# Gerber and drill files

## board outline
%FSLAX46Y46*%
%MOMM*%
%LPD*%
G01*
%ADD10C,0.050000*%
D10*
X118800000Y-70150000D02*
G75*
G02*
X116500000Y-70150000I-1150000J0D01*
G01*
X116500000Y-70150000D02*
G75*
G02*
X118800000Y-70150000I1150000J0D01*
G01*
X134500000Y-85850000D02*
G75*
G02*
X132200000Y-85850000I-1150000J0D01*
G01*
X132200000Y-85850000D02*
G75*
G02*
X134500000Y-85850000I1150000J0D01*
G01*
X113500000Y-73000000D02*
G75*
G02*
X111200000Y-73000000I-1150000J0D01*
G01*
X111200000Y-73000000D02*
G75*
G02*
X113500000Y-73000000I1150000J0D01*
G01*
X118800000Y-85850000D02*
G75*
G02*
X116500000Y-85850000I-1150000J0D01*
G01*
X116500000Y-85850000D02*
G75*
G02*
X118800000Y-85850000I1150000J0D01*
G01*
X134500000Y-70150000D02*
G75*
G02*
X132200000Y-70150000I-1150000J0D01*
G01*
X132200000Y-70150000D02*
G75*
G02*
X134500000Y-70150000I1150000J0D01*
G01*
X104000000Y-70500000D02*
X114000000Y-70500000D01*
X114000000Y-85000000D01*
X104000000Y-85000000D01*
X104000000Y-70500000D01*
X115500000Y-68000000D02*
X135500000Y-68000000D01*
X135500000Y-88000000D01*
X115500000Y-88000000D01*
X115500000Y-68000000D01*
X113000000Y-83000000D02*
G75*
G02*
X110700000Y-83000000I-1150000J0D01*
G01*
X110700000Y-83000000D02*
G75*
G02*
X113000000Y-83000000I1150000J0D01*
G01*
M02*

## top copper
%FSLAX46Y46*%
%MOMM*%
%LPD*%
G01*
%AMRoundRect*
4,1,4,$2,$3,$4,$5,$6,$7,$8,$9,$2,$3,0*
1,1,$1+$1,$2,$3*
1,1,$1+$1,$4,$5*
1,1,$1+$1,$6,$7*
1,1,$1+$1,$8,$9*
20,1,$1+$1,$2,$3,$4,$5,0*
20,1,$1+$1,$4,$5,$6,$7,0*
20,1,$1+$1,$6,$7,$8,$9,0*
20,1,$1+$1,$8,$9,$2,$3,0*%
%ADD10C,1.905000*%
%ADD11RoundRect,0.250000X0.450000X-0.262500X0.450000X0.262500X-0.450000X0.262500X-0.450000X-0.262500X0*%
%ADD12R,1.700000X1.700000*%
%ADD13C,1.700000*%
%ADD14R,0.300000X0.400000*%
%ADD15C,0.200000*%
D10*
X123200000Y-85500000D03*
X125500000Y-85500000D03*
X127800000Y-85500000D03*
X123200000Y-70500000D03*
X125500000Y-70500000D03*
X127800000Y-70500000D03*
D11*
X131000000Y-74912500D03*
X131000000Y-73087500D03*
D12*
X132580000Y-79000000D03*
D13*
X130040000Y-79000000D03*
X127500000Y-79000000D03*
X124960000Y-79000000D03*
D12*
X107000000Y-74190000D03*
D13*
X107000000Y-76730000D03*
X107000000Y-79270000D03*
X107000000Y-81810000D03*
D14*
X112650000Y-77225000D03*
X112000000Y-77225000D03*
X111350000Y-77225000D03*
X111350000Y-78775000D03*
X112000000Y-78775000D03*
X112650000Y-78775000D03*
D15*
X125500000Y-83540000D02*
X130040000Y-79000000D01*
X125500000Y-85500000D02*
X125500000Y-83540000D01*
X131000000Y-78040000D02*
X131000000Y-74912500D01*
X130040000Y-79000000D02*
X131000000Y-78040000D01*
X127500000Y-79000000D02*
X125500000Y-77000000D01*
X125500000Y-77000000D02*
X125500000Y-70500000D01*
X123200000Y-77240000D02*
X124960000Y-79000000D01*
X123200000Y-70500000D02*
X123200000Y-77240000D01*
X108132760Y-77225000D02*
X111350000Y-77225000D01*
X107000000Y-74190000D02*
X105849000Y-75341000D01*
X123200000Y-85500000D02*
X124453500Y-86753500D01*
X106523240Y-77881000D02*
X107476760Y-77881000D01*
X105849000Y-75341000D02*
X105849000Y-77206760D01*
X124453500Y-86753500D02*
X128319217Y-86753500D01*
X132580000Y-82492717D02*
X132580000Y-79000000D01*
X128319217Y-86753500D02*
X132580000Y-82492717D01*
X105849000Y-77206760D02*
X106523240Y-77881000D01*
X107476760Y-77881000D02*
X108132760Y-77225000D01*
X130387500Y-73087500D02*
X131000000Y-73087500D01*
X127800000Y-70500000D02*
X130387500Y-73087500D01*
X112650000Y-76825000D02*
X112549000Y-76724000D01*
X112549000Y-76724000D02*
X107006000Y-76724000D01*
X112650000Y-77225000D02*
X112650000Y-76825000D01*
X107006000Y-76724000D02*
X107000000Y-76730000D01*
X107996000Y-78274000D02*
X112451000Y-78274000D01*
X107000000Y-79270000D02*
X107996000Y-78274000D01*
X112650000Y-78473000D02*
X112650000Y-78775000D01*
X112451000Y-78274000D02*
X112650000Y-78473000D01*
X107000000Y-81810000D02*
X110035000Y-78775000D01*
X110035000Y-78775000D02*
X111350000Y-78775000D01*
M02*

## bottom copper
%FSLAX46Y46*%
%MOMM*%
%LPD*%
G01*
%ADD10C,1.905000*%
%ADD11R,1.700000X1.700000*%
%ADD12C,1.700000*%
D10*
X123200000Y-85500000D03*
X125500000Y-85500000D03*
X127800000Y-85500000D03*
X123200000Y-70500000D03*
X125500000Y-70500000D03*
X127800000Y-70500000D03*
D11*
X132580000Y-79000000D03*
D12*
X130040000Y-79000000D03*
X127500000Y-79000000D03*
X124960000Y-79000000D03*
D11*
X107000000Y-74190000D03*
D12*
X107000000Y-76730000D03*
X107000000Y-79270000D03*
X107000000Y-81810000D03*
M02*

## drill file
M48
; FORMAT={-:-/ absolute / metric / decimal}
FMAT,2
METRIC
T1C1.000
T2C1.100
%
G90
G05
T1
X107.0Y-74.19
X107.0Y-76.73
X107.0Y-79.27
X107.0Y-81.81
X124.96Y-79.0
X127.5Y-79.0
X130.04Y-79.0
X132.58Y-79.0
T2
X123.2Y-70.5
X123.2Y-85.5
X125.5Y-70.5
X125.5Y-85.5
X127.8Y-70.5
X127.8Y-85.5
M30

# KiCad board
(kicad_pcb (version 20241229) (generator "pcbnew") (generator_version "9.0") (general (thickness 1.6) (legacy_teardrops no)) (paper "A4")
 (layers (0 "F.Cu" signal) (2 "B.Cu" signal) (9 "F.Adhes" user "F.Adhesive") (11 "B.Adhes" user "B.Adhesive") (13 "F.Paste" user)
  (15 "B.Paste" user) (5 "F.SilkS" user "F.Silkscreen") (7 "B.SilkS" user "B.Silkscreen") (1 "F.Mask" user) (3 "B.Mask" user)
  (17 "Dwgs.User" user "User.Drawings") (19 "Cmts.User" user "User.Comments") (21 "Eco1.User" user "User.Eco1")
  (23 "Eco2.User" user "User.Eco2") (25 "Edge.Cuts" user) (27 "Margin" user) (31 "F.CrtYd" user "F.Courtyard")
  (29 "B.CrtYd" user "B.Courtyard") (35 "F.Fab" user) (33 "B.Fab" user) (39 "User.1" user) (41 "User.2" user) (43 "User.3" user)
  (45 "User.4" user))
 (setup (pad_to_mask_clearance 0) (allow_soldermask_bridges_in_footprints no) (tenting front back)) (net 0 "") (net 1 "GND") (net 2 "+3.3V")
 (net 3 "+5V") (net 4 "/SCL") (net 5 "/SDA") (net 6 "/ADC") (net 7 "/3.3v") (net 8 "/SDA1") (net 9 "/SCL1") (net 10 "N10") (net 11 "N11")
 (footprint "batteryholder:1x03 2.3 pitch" (layer "F.Cu") (at 123.4 85.5)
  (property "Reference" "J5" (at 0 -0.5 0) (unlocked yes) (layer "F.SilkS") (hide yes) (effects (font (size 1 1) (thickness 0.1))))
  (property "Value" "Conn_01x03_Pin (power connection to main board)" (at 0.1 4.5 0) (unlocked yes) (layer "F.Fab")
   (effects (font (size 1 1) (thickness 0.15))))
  (pad "1" thru_hole circle (at -0.2 0) (size 1.905 1.905) (drill 1.1) (layers "*.Cu" "*.Mask") (remove_unused_layers no) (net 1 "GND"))
  (pad "2" thru_hole circle (at 2.1 0) (size 1.905 1.905) (drill 1.1) (layers "*.Cu" "*.Mask") (remove_unused_layers no) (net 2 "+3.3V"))
  (pad "3" thru_hole circle (at 4.4 0) (size 1.905 1.905) (drill 1.1) (layers "*.Cu" "*.Mask") (remove_unused_layers no) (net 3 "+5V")))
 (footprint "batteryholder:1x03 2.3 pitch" (layer "F.Cu") (at 122.9 70.5)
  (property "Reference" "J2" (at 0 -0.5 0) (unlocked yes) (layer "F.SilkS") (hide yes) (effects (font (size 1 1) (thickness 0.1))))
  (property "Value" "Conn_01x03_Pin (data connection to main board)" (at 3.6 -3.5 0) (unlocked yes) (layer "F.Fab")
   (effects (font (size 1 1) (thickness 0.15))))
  (pad "1" thru_hole circle (at 0.3 0) (size 1.905 1.905) (drill 1.1) (layers "*.Cu" "*.Mask") (remove_unused_layers no) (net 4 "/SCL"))
  (pad "2" thru_hole circle (at 2.6 0) (size 1.905 1.905) (drill 1.1) (layers "*.Cu" "*.Mask") (remove_unused_layers no) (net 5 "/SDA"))
  (pad "3" thru_hole circle (at 4.9 0) (size 1.905 1.905) (drill 1.1) (layers "*.Cu" "*.Mask") (remove_unused_layers no) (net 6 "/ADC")))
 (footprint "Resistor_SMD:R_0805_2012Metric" (layer "F.Cu") (at 131 74 90)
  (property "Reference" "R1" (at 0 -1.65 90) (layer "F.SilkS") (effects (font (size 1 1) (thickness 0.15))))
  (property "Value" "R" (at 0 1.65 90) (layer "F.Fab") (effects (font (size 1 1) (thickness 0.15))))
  (pad "1" smd roundrect (at -0.9125 0 90) (size 1.025 1.4) (layers "F.Cu" "F.Mask" "F.Paste") (roundrect_rratio 0.243902) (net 2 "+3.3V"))
  (pad "2" smd roundrect (at 0.9125 0 90) (size 1.025 1.4) (layers "F.Cu" "F.Mask" "F.Paste") (roundrect_rratio 0.243902) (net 6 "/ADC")))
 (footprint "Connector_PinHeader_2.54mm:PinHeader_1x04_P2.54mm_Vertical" (layer "F.Cu") (at 132.58 79 -90)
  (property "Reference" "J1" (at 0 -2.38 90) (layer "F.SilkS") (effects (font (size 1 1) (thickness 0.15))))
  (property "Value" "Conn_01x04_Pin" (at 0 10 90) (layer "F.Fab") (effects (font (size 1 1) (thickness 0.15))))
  (pad "1" thru_hole rect (at 0 0 270) (size 1.7 1.7) (drill 1) (layers "*.Cu" "*.Mask") (remove_unused_layers no) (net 1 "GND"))
  (pad "2" thru_hole circle (at 0 2.54 270) (size 1.7 1.7) (drill 1) (layers "*.Cu" "*.Mask") (remove_unused_layers no) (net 2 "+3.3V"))
  (pad "3" thru_hole circle (at 0 5.08 270) (size 1.7 1.7) (drill 1) (layers "*.Cu" "*.Mask") (remove_unused_layers no) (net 5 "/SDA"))
  (pad "4" thru_hole circle (at 0 7.62 270) (size 1.7 1.7) (drill 1) (layers "*.Cu" "*.Mask") (remove_unused_layers no) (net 4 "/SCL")))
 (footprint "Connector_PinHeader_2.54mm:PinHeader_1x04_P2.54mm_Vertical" (layer "F.Cu") (at 107 74.19)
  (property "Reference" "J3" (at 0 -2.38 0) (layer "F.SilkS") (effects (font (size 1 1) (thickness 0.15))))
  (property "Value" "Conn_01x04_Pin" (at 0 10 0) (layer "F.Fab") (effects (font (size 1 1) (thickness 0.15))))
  (pad "1" thru_hole rect (at 0 0) (size 1.7 1.7) (drill 1) (layers "*.Cu" "*.Mask") (remove_unused_layers no) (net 1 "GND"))
  (pad "2" thru_hole circle (at 0 2.54) (size 1.7 1.7) (drill 1) (layers "*.Cu" "*.Mask") (remove_unused_layers no) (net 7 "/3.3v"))
  (pad "3" thru_hole circle (at 0 5.08) (size 1.7 1.7) (drill 1) (layers "*.Cu" "*.Mask") (remove_unused_layers no) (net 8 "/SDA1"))
  (pad "4" thru_hole circle (at 0 7.62) (size 1.7 1.7) (drill 1) (layers "*.Cu" "*.Mask") (remove_unused_layers no) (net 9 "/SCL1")))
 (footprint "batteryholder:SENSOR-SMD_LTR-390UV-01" (layer "F.Cu") (at 112 78 180)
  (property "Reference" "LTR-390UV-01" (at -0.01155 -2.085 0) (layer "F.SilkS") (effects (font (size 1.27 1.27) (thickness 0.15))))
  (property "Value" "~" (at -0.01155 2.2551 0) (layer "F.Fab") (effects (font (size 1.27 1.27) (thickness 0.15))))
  (pad "1" smd rect (at -0.65 0.775 180) (size 0.3 0.4) (layers "F.Cu" "F.Mask" "F.Paste") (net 7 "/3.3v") (solder_mask_margin 0.0508)
   (solder_paste_margin 0) (thermal_bridge_angle 0))
  (pad "2" smd rect (at 0 0.775 180) (size 0.3 0.4) (layers "F.Cu" "F.Mask" "F.Paste") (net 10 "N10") (solder_mask_margin 0.0508)
   (solder_paste_margin 0) (thermal_bridge_angle 0))
  (pad "3" smd rect (at 0.65 0.775 180) (size 0.3 0.4) (layers "F.Cu" "F.Mask" "F.Paste") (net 1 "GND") (solder_mask_margin 0.0508)
   (solder_paste_margin 0) (thermal_bridge_angle 0))
  (pad "4" smd rect (at 0.65 -0.775 180) (size 0.3 0.4) (layers "F.Cu" "F.Mask" "F.Paste") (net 9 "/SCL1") (solder_mask_margin 0.0508)
   (solder_paste_margin 0) (thermal_bridge_angle 0))
  (pad "5" smd rect (at 0 -0.775 180) (size 0.3 0.4) (layers "F.Cu" "F.Mask" "F.Paste") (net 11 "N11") (solder_mask_margin 0.0508)
   (solder_paste_margin 0) (thermal_bridge_angle 0))
  (pad "6" smd rect (at -0.65 -0.775 180) (size 0.3 0.4) (layers "F.Cu" "F.Mask" "F.Paste") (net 8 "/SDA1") (solder_mask_margin 0.0508)
   (solder_paste_margin 0) (thermal_bridge_angle 0))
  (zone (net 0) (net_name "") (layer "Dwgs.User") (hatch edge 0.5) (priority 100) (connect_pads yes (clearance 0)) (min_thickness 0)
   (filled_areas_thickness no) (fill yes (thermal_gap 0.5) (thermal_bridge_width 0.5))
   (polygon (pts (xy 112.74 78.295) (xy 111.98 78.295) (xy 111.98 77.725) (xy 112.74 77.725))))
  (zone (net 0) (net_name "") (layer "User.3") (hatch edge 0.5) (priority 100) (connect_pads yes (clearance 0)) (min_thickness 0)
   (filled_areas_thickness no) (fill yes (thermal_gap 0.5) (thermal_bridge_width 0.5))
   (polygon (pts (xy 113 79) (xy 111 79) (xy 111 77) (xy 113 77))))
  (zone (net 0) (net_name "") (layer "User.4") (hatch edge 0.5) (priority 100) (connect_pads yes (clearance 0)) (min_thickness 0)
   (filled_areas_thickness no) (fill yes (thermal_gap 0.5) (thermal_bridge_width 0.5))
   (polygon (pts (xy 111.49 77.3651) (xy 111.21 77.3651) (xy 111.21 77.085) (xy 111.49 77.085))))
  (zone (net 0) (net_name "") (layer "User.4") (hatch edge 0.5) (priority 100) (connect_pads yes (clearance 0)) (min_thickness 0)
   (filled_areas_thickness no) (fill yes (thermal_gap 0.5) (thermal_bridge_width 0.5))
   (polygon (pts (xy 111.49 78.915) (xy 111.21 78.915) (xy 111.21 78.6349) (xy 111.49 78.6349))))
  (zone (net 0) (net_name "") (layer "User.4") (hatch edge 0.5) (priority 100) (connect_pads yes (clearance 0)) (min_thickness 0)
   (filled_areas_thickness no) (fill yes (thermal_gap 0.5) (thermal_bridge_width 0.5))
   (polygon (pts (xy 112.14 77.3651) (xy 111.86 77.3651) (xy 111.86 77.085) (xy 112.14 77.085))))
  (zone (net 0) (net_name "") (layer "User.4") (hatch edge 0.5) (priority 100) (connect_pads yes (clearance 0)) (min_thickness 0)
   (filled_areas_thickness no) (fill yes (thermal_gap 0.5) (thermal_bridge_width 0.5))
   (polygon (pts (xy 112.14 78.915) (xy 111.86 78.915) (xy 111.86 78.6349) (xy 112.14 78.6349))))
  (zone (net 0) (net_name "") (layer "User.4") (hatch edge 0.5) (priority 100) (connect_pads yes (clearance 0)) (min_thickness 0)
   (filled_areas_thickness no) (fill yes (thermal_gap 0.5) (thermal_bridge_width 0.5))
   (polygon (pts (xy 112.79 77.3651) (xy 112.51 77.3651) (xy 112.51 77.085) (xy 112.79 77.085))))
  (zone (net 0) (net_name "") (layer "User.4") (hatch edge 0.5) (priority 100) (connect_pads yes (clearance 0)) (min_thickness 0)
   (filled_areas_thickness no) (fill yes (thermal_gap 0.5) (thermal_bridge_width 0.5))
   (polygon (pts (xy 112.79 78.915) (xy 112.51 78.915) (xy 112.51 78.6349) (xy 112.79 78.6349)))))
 (gr_circle (center 117.65 70.15) (end 118.8 70.15) (stroke (width 0.05) (type solid)) (fill no) (layer "Edge.Cuts"))
 (gr_circle (center 133.35 85.85) (end 134.5 85.85) (stroke (width 0.05) (type solid)) (fill no) (layer "Edge.Cuts"))
 (gr_circle (center 112.35 73) (end 113.5 73) (stroke (width 0.05) (type solid)) (fill no) (layer "Edge.Cuts"))
 (gr_circle (center 117.65 85.85) (end 118.8 85.85) (stroke (width 0.05) (type solid)) (fill no) (layer "Edge.Cuts"))
 (gr_circle (center 133.35 70.15) (end 134.5 70.15) (stroke (width 0.05) (type solid)) (fill no) (layer "Edge.Cuts"))
 (gr_rect (start 104 70.5) (end 114 85) (stroke (width 0.05) (type default)) (fill no) (layer "Edge.Cuts"))
 (gr_rect (start 115.5 68) (end 135.5 88) (stroke (width 0.05) (type solid)) (fill no) (layer "Edge.Cuts"))
 (gr_circle (center 111.85 83) (end 113 83) (stroke (width 0.05) (type solid)) (fill no) (layer "Edge.Cuts"))
 (segment (start 125.5 83.54) (end 130.04 79) (width 0.2) (layer "F.Cu") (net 2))
 (segment (start 125.5 85.5) (end 125.5 83.54) (width 0.2) (layer "F.Cu") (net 2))
 (segment (start 131 78.04) (end 131 74.9125) (width 0.2) (layer "F.Cu") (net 2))
 (segment (start 130.04 79) (end 131 78.04) (width 0.2) (layer "F.Cu") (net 2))
 (segment (start 127.5 79) (end 125.5 77) (width 0.2) (layer "F.Cu") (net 5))
 (segment (start 125.5 77) (end 125.5 70.5) (width 0.2) (layer "F.Cu") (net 5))
 (segment (start 123.2 77.24) (end 124.96 79) (width 0.2) (layer "F.Cu") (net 4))
 (segment (start 123.2 70.5) (end 123.2 77.24) (width 0.2) (layer "F.Cu") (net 4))
 (segment (start 108.13276 77.225) (end 111.35 77.225) (width 0.2) (layer "F.Cu") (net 1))
 (segment (start 107 74.19) (end 105.849 75.341) (width 0.2) (layer "F.Cu") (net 1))
 (segment (start 123.2 85.5) (end 124.4535 86.7535) (width 0.2) (layer "F.Cu") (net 1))
 (segment (start 106.52324 77.881) (end 107.47676 77.881) (width 0.2) (layer "F.Cu") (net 1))
 (segment (start 105.849 75.341) (end 105.849 77.20676) (width 0.2) (layer "F.Cu") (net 1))
 (segment (start 124.4535 86.7535) (end 128.319217 86.7535) (width 0.2) (layer "F.Cu") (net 1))
 (segment (start 132.58 82.492717) (end 132.58 79) (width 0.2) (layer "F.Cu") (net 1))
 (segment (start 128.319217 86.7535) (end 132.58 82.492717) (width 0.2) (layer "F.Cu") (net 1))
 (segment (start 105.849 77.20676) (end 106.52324 77.881) (width 0.2) (layer "F.Cu") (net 1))
 (segment (start 107.47676 77.881) (end 108.13276 77.225) (width 0.2) (layer "F.Cu") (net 1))
 (segment (start 130.3875 73.0875) (end 131 73.0875) (width 0.2) (layer "F.Cu") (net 6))
 (segment (start 127.8 70.5) (end 130.3875 73.0875) (width 0.2) (layer "F.Cu") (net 6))
 (segment (start 112.65 76.825) (end 112.549 76.724) (width 0.2) (layer "F.Cu") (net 7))
 (segment (start 112.549 76.724) (end 107.006 76.724) (width 0.2) (layer "F.Cu") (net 7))
 (segment (start 112.65 77.225) (end 112.65 76.825) (width 0.2) (layer "F.Cu") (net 7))
 (segment (start 107.006 76.724) (end 107 76.73) (width 0.2) (layer "F.Cu") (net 7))
 (segment (start 107.996 78.274) (end 112.451 78.274) (width 0.2) (layer "F.Cu") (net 8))
 (segment (start 107 79.27) (end 107.996 78.274) (width 0.2) (layer "F.Cu") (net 8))
 (segment (start 112.65 78.473) (end 112.65 78.775) (width 0.2) (layer "F.Cu") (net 8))
 (segment (start 112.451 78.274) (end 112.65 78.473) (width 0.2) (layer "F.Cu") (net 8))
 (segment (start 107 81.81) (end 110.035 78.775) (width 0.2) (layer "F.Cu") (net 9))
 (segment (start 110.035 78.775) (end 111.35 78.775) (width 0.2) (layer "F.Cu") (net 9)))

